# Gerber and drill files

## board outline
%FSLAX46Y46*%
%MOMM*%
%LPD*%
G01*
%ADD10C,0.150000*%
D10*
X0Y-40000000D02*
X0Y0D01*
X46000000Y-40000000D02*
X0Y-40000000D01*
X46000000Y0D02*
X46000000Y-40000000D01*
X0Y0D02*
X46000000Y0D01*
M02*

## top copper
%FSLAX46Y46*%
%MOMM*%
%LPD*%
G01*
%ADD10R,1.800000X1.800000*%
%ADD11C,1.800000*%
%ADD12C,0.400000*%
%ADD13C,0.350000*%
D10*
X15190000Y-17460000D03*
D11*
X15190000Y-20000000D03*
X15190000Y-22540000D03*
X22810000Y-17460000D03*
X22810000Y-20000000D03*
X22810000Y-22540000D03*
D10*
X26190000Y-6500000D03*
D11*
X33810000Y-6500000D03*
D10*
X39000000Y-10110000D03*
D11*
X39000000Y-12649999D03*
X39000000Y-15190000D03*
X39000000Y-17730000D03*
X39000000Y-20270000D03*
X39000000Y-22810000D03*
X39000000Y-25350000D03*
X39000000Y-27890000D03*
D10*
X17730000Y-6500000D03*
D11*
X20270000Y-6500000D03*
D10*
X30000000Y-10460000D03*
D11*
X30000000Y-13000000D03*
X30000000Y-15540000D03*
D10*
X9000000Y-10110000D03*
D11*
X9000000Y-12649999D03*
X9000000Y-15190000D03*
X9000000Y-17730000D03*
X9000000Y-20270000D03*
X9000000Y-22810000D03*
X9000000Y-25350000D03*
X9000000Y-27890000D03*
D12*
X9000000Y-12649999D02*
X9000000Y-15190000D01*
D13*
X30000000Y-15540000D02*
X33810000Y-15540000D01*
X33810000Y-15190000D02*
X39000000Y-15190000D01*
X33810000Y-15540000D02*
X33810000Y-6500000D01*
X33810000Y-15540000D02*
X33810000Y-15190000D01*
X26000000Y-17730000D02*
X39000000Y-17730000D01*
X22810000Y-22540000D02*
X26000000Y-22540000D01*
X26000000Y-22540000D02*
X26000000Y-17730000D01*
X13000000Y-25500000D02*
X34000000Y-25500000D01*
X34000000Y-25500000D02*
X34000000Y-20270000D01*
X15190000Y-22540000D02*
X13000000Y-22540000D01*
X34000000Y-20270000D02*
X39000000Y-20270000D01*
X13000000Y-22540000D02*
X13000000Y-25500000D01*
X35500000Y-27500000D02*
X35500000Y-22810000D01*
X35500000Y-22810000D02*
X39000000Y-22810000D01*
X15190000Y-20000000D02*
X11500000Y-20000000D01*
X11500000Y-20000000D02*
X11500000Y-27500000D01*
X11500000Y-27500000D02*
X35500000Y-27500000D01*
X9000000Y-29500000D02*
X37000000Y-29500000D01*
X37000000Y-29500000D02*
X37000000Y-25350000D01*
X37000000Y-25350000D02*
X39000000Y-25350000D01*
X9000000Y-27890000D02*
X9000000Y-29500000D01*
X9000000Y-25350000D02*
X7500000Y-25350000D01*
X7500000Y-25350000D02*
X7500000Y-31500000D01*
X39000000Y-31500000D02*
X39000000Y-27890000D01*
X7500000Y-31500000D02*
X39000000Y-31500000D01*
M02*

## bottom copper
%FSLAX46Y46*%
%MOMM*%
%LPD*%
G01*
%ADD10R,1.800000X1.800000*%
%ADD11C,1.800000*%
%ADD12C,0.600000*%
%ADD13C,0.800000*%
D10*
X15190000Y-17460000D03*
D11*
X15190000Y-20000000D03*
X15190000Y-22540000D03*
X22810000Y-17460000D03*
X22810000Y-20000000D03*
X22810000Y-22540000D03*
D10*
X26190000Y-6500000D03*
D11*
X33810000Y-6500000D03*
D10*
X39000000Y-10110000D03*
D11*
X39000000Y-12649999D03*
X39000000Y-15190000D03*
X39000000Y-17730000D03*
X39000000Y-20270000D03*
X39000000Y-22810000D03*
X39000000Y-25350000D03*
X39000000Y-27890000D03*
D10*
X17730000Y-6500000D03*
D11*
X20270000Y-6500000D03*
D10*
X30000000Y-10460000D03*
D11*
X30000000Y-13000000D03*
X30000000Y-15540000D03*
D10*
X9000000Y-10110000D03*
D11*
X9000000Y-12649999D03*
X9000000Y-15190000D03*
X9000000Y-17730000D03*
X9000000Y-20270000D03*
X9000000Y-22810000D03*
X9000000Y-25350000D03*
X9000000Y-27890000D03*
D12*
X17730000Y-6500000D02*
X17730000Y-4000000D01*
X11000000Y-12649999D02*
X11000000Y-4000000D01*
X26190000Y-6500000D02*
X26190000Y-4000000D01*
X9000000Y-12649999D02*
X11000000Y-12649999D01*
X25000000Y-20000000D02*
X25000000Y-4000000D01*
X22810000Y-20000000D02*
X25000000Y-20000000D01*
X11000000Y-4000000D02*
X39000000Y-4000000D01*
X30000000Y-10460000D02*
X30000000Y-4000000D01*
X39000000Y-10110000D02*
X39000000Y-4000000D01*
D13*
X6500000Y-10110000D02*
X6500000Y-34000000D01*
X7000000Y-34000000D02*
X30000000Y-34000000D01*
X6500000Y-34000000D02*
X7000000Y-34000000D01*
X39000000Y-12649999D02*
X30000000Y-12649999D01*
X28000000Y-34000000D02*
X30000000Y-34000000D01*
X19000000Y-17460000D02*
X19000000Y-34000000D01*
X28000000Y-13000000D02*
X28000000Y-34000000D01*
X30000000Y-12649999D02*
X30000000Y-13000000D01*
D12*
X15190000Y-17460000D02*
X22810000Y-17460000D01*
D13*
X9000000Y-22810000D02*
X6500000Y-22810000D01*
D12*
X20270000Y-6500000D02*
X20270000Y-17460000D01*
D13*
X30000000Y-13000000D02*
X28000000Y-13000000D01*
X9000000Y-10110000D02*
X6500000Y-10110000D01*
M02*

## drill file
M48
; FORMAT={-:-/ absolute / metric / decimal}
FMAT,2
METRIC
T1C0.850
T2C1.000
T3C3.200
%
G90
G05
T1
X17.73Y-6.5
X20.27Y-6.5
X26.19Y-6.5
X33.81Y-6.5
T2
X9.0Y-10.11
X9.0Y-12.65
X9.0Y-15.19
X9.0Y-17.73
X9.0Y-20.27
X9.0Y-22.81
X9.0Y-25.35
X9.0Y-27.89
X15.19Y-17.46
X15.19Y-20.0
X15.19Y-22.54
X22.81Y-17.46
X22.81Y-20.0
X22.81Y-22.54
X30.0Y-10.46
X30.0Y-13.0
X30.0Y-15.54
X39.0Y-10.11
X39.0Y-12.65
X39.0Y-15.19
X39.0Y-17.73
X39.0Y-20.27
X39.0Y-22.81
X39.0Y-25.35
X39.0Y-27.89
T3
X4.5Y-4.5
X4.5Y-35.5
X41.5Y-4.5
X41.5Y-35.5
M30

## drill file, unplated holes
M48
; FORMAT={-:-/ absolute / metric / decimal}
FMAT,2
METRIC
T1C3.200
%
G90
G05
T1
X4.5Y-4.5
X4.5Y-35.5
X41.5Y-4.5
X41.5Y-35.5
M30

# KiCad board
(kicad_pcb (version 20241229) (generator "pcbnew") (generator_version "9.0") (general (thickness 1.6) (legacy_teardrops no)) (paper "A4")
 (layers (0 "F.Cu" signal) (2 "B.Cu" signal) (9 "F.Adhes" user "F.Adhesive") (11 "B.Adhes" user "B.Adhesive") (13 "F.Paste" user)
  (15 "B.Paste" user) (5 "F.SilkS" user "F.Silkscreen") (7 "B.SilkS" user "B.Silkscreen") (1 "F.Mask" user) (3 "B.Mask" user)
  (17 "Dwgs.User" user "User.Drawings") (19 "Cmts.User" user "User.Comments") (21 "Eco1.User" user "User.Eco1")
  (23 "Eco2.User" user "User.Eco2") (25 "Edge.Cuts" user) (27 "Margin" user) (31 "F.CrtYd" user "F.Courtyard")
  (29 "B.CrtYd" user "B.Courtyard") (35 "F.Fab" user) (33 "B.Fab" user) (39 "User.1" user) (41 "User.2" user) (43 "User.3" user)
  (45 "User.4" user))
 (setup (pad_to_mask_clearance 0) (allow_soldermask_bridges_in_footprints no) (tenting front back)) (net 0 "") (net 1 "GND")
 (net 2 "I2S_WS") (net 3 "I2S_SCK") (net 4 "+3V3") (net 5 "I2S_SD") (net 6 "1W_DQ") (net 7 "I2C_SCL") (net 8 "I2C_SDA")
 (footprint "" (layer "F.Cu") (at 19 20)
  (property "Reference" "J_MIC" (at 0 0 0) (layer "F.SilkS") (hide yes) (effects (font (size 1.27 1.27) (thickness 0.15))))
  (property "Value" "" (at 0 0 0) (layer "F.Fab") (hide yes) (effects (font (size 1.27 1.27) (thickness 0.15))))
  (pad "1" thru_hole rect (at -3.81 -2.54) (size 1.8 1.8) (drill 1) (layers "*.Cu" "*.Mask") (remove_unused_layers no) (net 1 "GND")
   (thermal_bridge_angle 45))
  (pad "2" thru_hole circle (at -3.81 0) (size 1.8 1.8) (drill 1) (layers "*.Cu" "*.Mask") (remove_unused_layers no) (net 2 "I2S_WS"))
  (pad "3" thru_hole circle (at -3.81 2.54) (size 1.8 1.8) (drill 1) (layers "*.Cu" "*.Mask") (remove_unused_layers no) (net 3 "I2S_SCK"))
  (pad "4" thru_hole circle (at 3.81 -2.54) (size 1.8 1.8) (drill 1) (layers "*.Cu" "*.Mask") (remove_unused_layers no) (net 1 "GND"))
  (pad "5" thru_hole circle (at 3.81 0) (size 1.8 1.8) (drill 1) (layers "*.Cu" "*.Mask") (remove_unused_layers no) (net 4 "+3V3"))
  (pad "6" thru_hole circle (at 3.81 2.54) (size 1.8 1.8) (drill 1) (layers "*.Cu" "*.Mask") (remove_unused_layers no) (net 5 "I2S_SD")))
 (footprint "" (layer "F.Cu") (at 30 6.5)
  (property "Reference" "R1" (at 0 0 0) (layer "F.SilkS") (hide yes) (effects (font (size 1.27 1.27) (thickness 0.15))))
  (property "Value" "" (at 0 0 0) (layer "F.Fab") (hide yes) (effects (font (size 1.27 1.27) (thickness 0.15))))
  (pad "1" thru_hole rect (at -3.81 0) (size 1.8 1.8) (drill 0.85) (layers "*.Cu" "*.Mask") (remove_unused_layers no) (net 4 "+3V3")
   (thermal_bridge_angle 45))
  (pad "2" thru_hole circle (at 3.81 0) (size 1.8 1.8) (drill 0.85) (layers "*.Cu" "*.Mask") (remove_unused_layers no) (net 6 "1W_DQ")))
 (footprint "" (layer "F.Cu") (at 39 19)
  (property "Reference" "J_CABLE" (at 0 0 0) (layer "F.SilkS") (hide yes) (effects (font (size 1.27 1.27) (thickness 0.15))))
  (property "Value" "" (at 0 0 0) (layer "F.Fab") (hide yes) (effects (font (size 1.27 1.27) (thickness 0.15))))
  (pad "1" thru_hole rect (at 0 -8.89) (size 1.8 1.8) (drill 1) (layers "*.Cu" "*.Mask") (remove_unused_layers no) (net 4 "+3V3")
   (thermal_bridge_angle 45))
  (pad "2" thru_hole circle (at 0 -6.350001) (size 1.8 1.8) (drill 1) (layers "*.Cu" "*.Mask") (remove_unused_layers no) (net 1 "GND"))
  (pad "3" thru_hole circle (at 0 -3.81) (size 1.8 1.8) (drill 1) (layers "*.Cu" "*.Mask") (remove_unused_layers no) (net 6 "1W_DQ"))
  (pad "4" thru_hole circle (at 0 -1.27) (size 1.8 1.8) (drill 1) (layers "*.Cu" "*.Mask") (remove_unused_layers no) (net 5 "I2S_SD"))
  (pad "5" thru_hole circle (at 0 1.27) (size 1.8 1.8) (drill 1) (layers "*.Cu" "*.Mask") (remove_unused_layers no) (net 3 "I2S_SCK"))
  (pad "6" thru_hole circle (at 0 3.81) (size 1.8 1.8) (drill 1) (layers "*.Cu" "*.Mask") (remove_unused_layers no) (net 2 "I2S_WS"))
  (pad "7" thru_hole circle (at 0 6.35) (size 1.8 1.8) (drill 1) (layers "*.Cu" "*.Mask") (remove_unused_layers no) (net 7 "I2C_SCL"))
  (pad "8" thru_hole circle (at 0 8.89) (size 1.8 1.8) (drill 1) (layers "*.Cu" "*.Mask") (remove_unused_layers no) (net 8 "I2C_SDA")))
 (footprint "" (layer "F.Cu") (at 19 6.5)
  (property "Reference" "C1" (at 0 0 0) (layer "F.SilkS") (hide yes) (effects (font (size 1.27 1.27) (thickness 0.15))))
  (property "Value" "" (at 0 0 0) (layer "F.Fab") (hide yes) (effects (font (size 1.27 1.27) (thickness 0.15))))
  (pad "1" thru_hole rect (at -1.27 0) (size 1.8 1.8) (drill 0.85) (layers "*.Cu" "*.Mask") (remove_unused_layers no) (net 4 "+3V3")
   (thermal_bridge_angle 45))
  (pad "2" thru_hole circle (at 1.27 0) (size 1.8 1.8) (drill 0.85) (layers "*.Cu" "*.Mask") (remove_unused_layers no) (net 1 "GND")))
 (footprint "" (layer "F.Cu") (at 30 13)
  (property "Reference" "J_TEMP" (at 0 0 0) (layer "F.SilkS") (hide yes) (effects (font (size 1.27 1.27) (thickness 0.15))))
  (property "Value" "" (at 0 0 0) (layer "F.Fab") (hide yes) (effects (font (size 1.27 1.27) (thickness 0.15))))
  (pad "1" thru_hole rect (at 0 -2.54) (size 1.8 1.8) (drill 1) (layers "*.Cu" "*.Mask") (remove_unused_layers no) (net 4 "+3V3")
   (thermal_bridge_angle 45))
  (pad "2" thru_hole circle (at 0 0) (size 1.8 1.8) (drill 1) (layers "*.Cu" "*.Mask") (remove_unused_layers no) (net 1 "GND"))
  (pad "3" thru_hole circle (at 0 2.54) (size 1.8 1.8) (drill 1) (layers "*.Cu" "*.Mask") (remove_unused_layers no) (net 6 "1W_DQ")))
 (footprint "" (layer "F.Cu") (at 4.5 4.5)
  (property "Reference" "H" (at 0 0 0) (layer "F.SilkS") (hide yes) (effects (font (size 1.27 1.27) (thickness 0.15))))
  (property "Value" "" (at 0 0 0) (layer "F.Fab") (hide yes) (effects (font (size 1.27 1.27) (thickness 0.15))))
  (pad "" np_thru_hole circle (at 0 0) (size 3.2 3.2) (drill 3.2) (layers "*.Cu" "*.Mask")))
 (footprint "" (layer "F.Cu") (at 41.5 4.5)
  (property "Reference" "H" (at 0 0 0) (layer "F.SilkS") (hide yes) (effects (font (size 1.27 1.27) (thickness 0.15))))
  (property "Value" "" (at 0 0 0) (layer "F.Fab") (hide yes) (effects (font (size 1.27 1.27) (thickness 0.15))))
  (pad "" np_thru_hole circle (at 0 0) (size 3.2 3.2) (drill 3.2) (layers "*.Cu" "*.Mask")))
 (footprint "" (layer "F.Cu") (at 4.5 35.5)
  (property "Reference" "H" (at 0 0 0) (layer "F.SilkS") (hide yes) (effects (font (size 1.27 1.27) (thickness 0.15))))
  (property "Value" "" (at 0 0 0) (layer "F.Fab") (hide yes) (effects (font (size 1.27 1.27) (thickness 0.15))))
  (pad "" np_thru_hole circle (at 0 0) (size 3.2 3.2) (drill 3.2) (layers "*.Cu" "*.Mask")))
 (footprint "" (layer "F.Cu") (at 9 19)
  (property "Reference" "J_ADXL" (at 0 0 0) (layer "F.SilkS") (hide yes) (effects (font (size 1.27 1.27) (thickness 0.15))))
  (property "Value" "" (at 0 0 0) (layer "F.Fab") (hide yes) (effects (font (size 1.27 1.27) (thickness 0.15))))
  (pad "1" thru_hole rect (at 0 -8.89) (size 1.8 1.8) (drill 1) (layers "*.Cu" "*.Mask") (remove_unused_layers no) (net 1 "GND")
   (thermal_bridge_angle 45))
  (pad "2" thru_hole circle (at 0 -6.350001) (size 1.8 1.8) (drill 1) (layers "*.Cu" "*.Mask") (remove_unused_layers no) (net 4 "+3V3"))
  (pad "3" thru_hole circle (at 0 -3.81) (size 1.8 1.8) (drill 1) (layers "*.Cu" "*.Mask") (remove_unused_layers no) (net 4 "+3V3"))
  (pad "4" thru_hole circle (at 0 -1.27) (size 1.8 1.8) (drill 1) (layers "*.Cu" "*.Mask") (remove_unused_layers no))
  (pad "5" thru_hole circle (at 0 1.27) (size 1.8 1.8) (drill 1) (layers "*.Cu" "*.Mask") (remove_unused_layers no))
  (pad "6" thru_hole circle (at 0 3.81) (size 1.8 1.8) (drill 1) (layers "*.Cu" "*.Mask") (remove_unused_layers no) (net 1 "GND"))
  (pad "7" thru_hole circle (at 0 6.35) (size 1.8 1.8) (drill 1) (layers "*.Cu" "*.Mask") (remove_unused_layers no) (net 8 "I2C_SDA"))
  (pad "8" thru_hole circle (at 0 8.89) (size 1.8 1.8) (drill 1) (layers "*.Cu" "*.Mask") (remove_unused_layers no) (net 7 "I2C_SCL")))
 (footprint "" (layer "F.Cu") (at 41.5 35.5)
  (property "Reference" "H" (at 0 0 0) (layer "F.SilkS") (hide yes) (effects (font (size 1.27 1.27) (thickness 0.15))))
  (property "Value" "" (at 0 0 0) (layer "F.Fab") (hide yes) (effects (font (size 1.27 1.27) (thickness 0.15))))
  (pad "" np_thru_hole circle (at 0 0) (size 3.2 3.2) (drill 3.2) (layers "*.Cu" "*.Mask")))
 (gr_line (start 0 40) (end 0 0) (stroke (width 0.15) (type default)) (layer "Edge.Cuts"))
 (gr_line (start 46 40) (end 0 40) (stroke (width 0.15) (type default)) (layer "Edge.Cuts"))
 (gr_line (start 46 0) (end 46 40) (stroke (width 0.15) (type default)) (layer "Edge.Cuts"))
 (gr_line (start 0 0) (end 46 0) (stroke (width 0.15) (type default)) (layer "Edge.Cuts"))
 (segment (start 9 12.649999) (end 9 15.19) (width 0.4) (layer "F.Cu") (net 4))
 (segment (start 17.73 6.5) (end 17.73 4) (width 0.6) (layer "B.Cu") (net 4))
 (segment (start 11 12.649999) (end 11 4) (width 0.6) (layer "B.Cu") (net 4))
 (segment (start 26.19 6.5) (end 26.19 4) (width 0.6) (layer "B.Cu") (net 4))
 (segment (start 9 12.649999) (end 11 12.649999) (width 0.6) (layer "B.Cu") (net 4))
 (segment (start 25 20) (end 25 4) (width 0.6) (layer "B.Cu") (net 4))
 (segment (start 22.81 20) (end 25 20) (width 0.6) (layer "B.Cu") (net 4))
 (segment (start 11 4) (end 39 4) (width 0.6) (layer "B.Cu") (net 4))
 (segment (start 30 10.46) (end 30 4) (width 0.6) (layer "B.Cu") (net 4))
 (segment (start 39 10.11) (end 39 4) (width 0.6) (layer "B.Cu") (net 4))
 (segment (start 30 13) (end 28 13) (width 0.8) (layer "B.Cu") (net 1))
 (segment (start 6.5 10.11) (end 9 10.11) (width 0.8) (layer "B.Cu") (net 1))
 (segment (start 39 12.649999) (end 30 12.649999) (width 0.8) (layer "B.Cu") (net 1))
 (segment (start 28 34) (end 6.5 34) (width 0.8) (layer "B.Cu") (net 1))
 (segment (start 28 13) (end 28 34) (width 0.8) (layer "B.Cu") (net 1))
 (segment (start 30 12.649999) (end 30 13) (width 0.8) (layer "B.Cu") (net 1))
 (segment (start 15.19 17.46) (end 22.81 17.46) (width 0.6) (layer "B.Cu") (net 1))
 (segment (start 6.5 34) (end 6.5 10.11) (width 0.8) (layer "B.Cu") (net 1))
 (segment (start 9 22.81) (end 6.5 22.81) (width 0.8) (layer "B.Cu") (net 1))
 (segment (start 20.27 6.5) (end 20.27 17.46) (width 0.6) (layer "B.Cu") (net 1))
 (segment (start 19 17.46) (end 19 34) (width 0.8) (layer "B.Cu") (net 1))
 (segment (start 30 15.54) (end 33.81 15.54) (width 0.35) (layer "F.Cu") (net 6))
 (segment (start 33.81 15.19) (end 39 15.19) (width 0.35) (layer "F.Cu") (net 6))
 (segment (start 33.81 15.54) (end 33.81 6.5) (width 0.35) (layer "F.Cu") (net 6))
 (segment (start 33.81 15.54) (end 33.81 15.19) (width 0.35) (layer "F.Cu") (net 6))
 (segment (start 26 17.73) (end 39 17.73) (width 0.35) (layer "F.Cu") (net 5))
 (segment (start 22.81 22.54) (end 26 22.54) (width 0.35) (layer "F.Cu") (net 5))
 (segment (start 26 22.54) (end 26 17.73) (width 0.35) (layer "F.Cu") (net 5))
 (segment (start 13 25.5) (end 34 25.5) (width 0.35) (layer "F.Cu") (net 3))
 (segment (start 34 25.5) (end 34 20.27) (width 0.35) (layer "F.Cu") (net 3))
 (segment (start 15.19 22.54) (end 13 22.54) (width 0.35) (layer "F.Cu") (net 3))
 (segment (start 34 20.27) (end 39 20.27) (width 0.35) (layer "F.Cu") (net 3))
 (segment (start 13 22.54) (end 13 25.5) (width 0.35) (layer "F.Cu") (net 3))
 (segment (start 35.5 27.5) (end 35.5 22.81) (width 0.35) (layer "F.Cu") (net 2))
 (segment (start 35.5 22.81) (end 39 22.81) (width 0.35) (layer "F.Cu") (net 2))
 (segment (start 15.19 20) (end 11.5 20) (width 0.35) (layer "F.Cu") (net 2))
 (segment (start 11.5 20) (end 11.5 27.5) (width 0.35) (layer "F.Cu") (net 2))
 (segment (start 11.5 27.5) (end 35.5 27.5) (width 0.35) (layer "F.Cu") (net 2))
 (segment (start 9 29.5) (end 37 29.5) (width 0.35) (layer "F.Cu") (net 7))
 (segment (start 37 29.5) (end 37 25.35) (width 0.35) (layer "F.Cu") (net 7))
 (segment (start 37 25.35) (end 39 25.35) (width 0.35) (layer "F.Cu") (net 7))
 (segment (start 9 27.89) (end 9 29.5) (width 0.35) (layer "F.Cu") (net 7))
 (segment (start 9 25.35) (end 7.5 25.35) (width 0.35) (layer "F.Cu") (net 8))
 (segment (start 7.5 25.35) (end 7.5 31.5) (width 0.35) (layer "F.Cu") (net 8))
 (segment (start 39 31.5) (end 39 27.89) (width 0.35) (layer "F.Cu") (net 8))
 (segment (start 7.5 31.5) (end 39 31.5) (width 0.35) (layer "F.Cu") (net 8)))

